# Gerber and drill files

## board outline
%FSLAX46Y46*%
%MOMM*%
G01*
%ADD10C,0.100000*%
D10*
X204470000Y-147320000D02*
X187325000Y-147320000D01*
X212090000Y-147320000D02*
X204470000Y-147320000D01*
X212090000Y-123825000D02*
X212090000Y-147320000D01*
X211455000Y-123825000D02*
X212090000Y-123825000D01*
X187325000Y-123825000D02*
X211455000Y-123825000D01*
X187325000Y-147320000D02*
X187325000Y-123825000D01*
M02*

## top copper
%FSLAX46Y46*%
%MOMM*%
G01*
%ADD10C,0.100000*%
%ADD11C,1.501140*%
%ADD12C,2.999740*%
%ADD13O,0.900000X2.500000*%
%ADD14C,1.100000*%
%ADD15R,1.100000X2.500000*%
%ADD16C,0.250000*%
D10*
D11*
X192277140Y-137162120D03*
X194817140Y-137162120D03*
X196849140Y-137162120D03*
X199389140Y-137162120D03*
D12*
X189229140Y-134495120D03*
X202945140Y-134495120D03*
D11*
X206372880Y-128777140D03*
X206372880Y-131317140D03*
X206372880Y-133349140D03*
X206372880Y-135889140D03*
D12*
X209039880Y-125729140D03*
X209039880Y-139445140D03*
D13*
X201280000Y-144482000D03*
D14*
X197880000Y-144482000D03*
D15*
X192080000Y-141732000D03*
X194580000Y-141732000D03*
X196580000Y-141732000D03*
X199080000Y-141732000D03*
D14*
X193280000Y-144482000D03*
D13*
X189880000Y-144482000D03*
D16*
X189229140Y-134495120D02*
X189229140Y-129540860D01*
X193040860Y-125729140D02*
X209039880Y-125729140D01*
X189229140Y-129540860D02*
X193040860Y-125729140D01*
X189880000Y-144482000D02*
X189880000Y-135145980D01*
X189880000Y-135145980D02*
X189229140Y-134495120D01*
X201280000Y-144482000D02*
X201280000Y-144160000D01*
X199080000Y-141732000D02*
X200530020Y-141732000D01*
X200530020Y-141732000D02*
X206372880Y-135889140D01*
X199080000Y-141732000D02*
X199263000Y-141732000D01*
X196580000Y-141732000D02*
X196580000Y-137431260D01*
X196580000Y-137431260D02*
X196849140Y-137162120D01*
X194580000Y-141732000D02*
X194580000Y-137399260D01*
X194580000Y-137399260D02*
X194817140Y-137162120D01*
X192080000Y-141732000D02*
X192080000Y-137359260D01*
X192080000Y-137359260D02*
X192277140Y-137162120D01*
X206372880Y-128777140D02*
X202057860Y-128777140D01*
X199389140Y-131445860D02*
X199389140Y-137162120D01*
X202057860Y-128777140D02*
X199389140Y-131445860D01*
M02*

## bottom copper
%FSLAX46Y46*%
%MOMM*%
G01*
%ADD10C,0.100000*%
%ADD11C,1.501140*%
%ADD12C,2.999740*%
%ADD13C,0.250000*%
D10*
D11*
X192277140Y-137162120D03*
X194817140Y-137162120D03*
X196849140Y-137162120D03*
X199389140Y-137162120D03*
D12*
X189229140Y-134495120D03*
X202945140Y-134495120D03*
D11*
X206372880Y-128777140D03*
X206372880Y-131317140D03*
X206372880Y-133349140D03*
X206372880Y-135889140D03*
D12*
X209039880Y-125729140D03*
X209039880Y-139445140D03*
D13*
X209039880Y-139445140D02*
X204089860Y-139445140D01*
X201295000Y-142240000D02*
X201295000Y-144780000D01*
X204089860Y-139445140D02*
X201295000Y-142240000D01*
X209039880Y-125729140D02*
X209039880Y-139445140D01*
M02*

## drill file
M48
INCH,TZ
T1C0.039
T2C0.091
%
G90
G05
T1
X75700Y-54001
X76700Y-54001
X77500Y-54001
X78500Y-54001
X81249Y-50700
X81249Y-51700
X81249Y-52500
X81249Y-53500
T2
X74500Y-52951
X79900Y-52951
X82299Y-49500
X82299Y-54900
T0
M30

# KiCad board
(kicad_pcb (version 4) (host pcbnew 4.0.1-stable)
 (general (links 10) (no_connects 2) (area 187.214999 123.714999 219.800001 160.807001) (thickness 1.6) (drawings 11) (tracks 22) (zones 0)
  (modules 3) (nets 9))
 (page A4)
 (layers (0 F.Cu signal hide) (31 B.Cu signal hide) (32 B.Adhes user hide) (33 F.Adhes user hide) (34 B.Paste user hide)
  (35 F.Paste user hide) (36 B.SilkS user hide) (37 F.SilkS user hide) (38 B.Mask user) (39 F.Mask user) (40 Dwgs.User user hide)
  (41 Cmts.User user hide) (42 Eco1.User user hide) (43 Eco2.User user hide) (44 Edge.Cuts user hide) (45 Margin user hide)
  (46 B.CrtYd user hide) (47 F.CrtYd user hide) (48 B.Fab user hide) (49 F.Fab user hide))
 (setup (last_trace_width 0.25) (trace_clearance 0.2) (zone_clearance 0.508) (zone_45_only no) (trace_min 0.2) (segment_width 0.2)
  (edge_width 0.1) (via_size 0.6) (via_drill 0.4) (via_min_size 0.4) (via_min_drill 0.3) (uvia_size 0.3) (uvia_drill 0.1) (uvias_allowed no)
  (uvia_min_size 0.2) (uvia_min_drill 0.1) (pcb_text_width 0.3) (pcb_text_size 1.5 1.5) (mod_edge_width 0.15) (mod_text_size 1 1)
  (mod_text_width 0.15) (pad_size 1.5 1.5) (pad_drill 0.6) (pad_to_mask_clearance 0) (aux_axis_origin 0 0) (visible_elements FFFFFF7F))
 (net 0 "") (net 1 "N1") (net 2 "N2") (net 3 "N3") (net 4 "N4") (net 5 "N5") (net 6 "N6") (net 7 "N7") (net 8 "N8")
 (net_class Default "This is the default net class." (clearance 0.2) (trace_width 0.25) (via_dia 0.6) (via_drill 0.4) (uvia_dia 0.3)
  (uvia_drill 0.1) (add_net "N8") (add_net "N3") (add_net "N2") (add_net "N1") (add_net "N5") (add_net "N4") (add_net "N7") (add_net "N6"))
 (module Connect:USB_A (layer F.Cu) (at 199.39 137.16 180)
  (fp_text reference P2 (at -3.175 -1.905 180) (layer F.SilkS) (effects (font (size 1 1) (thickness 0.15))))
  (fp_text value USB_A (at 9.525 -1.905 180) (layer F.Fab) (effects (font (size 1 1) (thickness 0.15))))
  (pad 4 thru_hole circle (at 7.11286 -0.00212 90) (size 1.50114 1.50114) (drill 1.00076) (layers *.Cu *.Mask F.SilkS) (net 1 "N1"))
  (pad 3 thru_hole circle (at 4.57286 -0.00212 90) (size 1.50114 1.50114) (drill 1.00076) (layers *.Cu *.Mask F.SilkS) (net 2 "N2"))
  (pad 2 thru_hole circle (at 2.54086 -0.00212 90) (size 1.50114 1.50114) (drill 1.00076) (layers *.Cu *.Mask F.SilkS) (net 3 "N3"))
  (pad 1 thru_hole circle (at 0.00086 -0.00212 90) (size 1.50114 1.50114) (drill 1.00076) (layers *.Cu *.Mask F.SilkS) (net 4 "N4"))
  (pad 5 thru_hole circle (at 10.16086 2.66488 90) (size 2.99974 2.99974) (drill 2.30124) (layers *.Cu *.Mask F.SilkS) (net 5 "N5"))
  (pad 5 thru_hole circle (at -3.55514 2.66488 90) (size 2.99974 2.99974) (drill 2.30124) (layers *.Cu *.Mask F.SilkS) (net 5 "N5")))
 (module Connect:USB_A (layer F.Cu) (at 206.375 135.89 90)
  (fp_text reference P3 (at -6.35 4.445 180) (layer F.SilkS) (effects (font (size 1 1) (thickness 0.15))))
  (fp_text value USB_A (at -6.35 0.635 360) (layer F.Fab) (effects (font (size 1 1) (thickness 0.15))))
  (pad 4 thru_hole circle (at 7.11286 -0.00212) (size 1.50114 1.50114) (drill 1.00076) (layers *.Cu *.Mask F.SilkS) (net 4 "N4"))
  (pad 3 thru_hole circle (at 4.57286 -0.00212) (size 1.50114 1.50114) (drill 1.00076) (layers *.Cu *.Mask F.SilkS) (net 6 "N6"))
  (pad 2 thru_hole circle (at 2.54086 -0.00212) (size 1.50114 1.50114) (drill 1.00076) (layers *.Cu *.Mask F.SilkS) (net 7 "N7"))
  (pad 1 thru_hole circle (at 0.00086 -0.00212) (size 1.50114 1.50114) (drill 1.00076) (layers *.Cu *.Mask F.SilkS) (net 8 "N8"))
  (pad 5 thru_hole circle (at 10.16086 2.66488) (size 2.99974 2.99974) (drill 2.30124) (layers *.Cu *.Mask F.SilkS) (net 5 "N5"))
  (pad 5 thru_hole circle (at -3.55514 2.66488) (size 2.99974 2.99974) (drill 2.30124) (layers *.Cu *.Mask F.SilkS) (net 5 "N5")))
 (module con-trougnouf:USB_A (layer F.Cu) (at 195.58 146.05)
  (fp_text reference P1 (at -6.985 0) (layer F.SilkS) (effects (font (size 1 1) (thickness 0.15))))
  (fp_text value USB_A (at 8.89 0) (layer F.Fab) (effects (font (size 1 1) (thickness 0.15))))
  (pad 5 smd oval (at 5.7 -1.568) (size 0.9 2.5) (layers F.Cu F.Paste F.Mask) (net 5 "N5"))
  (pad "" smd circle (at 2.3 -1.568) (size 1.1 1.1) (layers F.Cu F.Paste F.Mask))
  (pad 4 smd rect (at -3.5 -4.318) (size 1.1 2.5) (layers F.Cu F.Paste F.Mask) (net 1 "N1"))
  (pad 3 smd rect (at -1 -4.318) (size 1.1 2.5) (layers F.Cu F.Paste F.Mask) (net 2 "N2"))
  (pad 2 smd rect (at 1 -4.318) (size 1.1 2.5) (layers F.Cu F.Paste F.Mask) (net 3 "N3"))
  (pad 1 smd rect (at 3.5 -4.318) (size 1.1 2.5) (layers F.Cu F.Paste F.Mask) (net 8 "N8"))
  (pad "" smd circle (at -2.3 -1.568) (size 1.1 1.1) (layers F.Cu F.Paste F.Mask))
  (pad 5 smd oval (at -5.7 -1.568) (size 0.9 2.5) (layers F.Cu F.Paste F.Mask) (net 5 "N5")))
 (gr_line (start 204.47 147.32) (end 187.325 147.32) (angle 90) (layer Edge.Cuts) (width 0.1))
 (gr_line (start 212.09 147.32) (end 204.47 147.32) (angle 90) (layer Edge.Cuts) (width 0.1))
 (gr_line (start 212.09 123.825) (end 212.09 147.32) (angle 90) (layer Edge.Cuts) (width 0.1))
 (gr_line (start 211.455 123.825) (end 212.09 123.825) (angle 90) (layer Edge.Cuts) (width 0.1))
 (gr_line (start 187.325 123.825) (end 211.455 123.825) (angle 90) (layer Edge.Cuts) (width 0.1))
 (gr_line (start 187.325 147.32) (end 187.325 123.825) (angle 90) (layer Edge.Cuts) (width 0.1))
 (segment (start 209.03988 139.44514) (end 204.08986 139.44514) (width 0.25) (layer B.Cu) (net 5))
 (segment (start 201.295 142.24) (end 201.295 144.78) (width 0.25) (layer B.Cu) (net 5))
 (segment (start 204.08986 139.44514) (end 201.295 142.24) (width 0.25) (layer B.Cu) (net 5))
 (segment (start 209.03988 125.72914) (end 209.03988 139.44514) (width 0.25) (layer B.Cu) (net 5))
 (segment (start 189.22914 134.49512) (end 189.22914 129.54086) (width 0.25) (layer F.Cu) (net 5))
 (segment (start 193.04086 125.72914) (end 209.03988 125.72914) (width 0.25) (layer F.Cu) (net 5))
 (segment (start 189.22914 129.54086) (end 193.04086 125.72914) (width 0.25) (layer F.Cu) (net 5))
 (segment (start 189.88 144.482) (end 189.88 135.14598) (width 0.25) (layer F.Cu) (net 5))
 (segment (start 189.88 135.14598) (end 189.22914 134.49512) (width 0.25) (layer F.Cu) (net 5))
 (segment (start 201.28 144.482) (end 201.28 144.16) (width 0.25) (layer F.Cu) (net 5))
 (segment (start 199.08 141.732) (end 200.53002 141.732) (width 0.25) (layer F.Cu) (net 8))
 (segment (start 200.53002 141.732) (end 206.37288 135.88914) (width 0.25) (layer F.Cu) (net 8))
 (segment (start 199.08 141.732) (end 199.263 141.732) (width 0.25) (layer F.Cu) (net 8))
 (segment (start 196.58 141.732) (end 196.58 137.43126) (width 0.25) (layer F.Cu) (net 3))
 (segment (start 196.58 137.43126) (end 196.84914 137.16212) (width 0.25) (layer F.Cu) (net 3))
 (segment (start 194.58 141.732) (end 194.58 137.39926) (width 0.25) (layer F.Cu) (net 2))
 (segment (start 194.58 137.39926) (end 194.81714 137.16212) (width 0.25) (layer F.Cu) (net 2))
 (segment (start 192.08 141.732) (end 192.08 137.35926) (width 0.25) (layer F.Cu) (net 1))
 (segment (start 192.08 137.35926) (end 192.27714 137.16212) (width 0.25) (layer F.Cu) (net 1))
 (segment (start 206.37288 128.77714) (end 202.05786 128.77714) (width 0.25) (layer F.Cu) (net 4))
 (segment (start 199.38914 131.44586) (end 199.38914 137.16212) (width 0.25) (layer F.Cu) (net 4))
 (segment (start 202.05786 128.77714) (end 199.38914 131.44586) (width 0.25) (layer F.Cu) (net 4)))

